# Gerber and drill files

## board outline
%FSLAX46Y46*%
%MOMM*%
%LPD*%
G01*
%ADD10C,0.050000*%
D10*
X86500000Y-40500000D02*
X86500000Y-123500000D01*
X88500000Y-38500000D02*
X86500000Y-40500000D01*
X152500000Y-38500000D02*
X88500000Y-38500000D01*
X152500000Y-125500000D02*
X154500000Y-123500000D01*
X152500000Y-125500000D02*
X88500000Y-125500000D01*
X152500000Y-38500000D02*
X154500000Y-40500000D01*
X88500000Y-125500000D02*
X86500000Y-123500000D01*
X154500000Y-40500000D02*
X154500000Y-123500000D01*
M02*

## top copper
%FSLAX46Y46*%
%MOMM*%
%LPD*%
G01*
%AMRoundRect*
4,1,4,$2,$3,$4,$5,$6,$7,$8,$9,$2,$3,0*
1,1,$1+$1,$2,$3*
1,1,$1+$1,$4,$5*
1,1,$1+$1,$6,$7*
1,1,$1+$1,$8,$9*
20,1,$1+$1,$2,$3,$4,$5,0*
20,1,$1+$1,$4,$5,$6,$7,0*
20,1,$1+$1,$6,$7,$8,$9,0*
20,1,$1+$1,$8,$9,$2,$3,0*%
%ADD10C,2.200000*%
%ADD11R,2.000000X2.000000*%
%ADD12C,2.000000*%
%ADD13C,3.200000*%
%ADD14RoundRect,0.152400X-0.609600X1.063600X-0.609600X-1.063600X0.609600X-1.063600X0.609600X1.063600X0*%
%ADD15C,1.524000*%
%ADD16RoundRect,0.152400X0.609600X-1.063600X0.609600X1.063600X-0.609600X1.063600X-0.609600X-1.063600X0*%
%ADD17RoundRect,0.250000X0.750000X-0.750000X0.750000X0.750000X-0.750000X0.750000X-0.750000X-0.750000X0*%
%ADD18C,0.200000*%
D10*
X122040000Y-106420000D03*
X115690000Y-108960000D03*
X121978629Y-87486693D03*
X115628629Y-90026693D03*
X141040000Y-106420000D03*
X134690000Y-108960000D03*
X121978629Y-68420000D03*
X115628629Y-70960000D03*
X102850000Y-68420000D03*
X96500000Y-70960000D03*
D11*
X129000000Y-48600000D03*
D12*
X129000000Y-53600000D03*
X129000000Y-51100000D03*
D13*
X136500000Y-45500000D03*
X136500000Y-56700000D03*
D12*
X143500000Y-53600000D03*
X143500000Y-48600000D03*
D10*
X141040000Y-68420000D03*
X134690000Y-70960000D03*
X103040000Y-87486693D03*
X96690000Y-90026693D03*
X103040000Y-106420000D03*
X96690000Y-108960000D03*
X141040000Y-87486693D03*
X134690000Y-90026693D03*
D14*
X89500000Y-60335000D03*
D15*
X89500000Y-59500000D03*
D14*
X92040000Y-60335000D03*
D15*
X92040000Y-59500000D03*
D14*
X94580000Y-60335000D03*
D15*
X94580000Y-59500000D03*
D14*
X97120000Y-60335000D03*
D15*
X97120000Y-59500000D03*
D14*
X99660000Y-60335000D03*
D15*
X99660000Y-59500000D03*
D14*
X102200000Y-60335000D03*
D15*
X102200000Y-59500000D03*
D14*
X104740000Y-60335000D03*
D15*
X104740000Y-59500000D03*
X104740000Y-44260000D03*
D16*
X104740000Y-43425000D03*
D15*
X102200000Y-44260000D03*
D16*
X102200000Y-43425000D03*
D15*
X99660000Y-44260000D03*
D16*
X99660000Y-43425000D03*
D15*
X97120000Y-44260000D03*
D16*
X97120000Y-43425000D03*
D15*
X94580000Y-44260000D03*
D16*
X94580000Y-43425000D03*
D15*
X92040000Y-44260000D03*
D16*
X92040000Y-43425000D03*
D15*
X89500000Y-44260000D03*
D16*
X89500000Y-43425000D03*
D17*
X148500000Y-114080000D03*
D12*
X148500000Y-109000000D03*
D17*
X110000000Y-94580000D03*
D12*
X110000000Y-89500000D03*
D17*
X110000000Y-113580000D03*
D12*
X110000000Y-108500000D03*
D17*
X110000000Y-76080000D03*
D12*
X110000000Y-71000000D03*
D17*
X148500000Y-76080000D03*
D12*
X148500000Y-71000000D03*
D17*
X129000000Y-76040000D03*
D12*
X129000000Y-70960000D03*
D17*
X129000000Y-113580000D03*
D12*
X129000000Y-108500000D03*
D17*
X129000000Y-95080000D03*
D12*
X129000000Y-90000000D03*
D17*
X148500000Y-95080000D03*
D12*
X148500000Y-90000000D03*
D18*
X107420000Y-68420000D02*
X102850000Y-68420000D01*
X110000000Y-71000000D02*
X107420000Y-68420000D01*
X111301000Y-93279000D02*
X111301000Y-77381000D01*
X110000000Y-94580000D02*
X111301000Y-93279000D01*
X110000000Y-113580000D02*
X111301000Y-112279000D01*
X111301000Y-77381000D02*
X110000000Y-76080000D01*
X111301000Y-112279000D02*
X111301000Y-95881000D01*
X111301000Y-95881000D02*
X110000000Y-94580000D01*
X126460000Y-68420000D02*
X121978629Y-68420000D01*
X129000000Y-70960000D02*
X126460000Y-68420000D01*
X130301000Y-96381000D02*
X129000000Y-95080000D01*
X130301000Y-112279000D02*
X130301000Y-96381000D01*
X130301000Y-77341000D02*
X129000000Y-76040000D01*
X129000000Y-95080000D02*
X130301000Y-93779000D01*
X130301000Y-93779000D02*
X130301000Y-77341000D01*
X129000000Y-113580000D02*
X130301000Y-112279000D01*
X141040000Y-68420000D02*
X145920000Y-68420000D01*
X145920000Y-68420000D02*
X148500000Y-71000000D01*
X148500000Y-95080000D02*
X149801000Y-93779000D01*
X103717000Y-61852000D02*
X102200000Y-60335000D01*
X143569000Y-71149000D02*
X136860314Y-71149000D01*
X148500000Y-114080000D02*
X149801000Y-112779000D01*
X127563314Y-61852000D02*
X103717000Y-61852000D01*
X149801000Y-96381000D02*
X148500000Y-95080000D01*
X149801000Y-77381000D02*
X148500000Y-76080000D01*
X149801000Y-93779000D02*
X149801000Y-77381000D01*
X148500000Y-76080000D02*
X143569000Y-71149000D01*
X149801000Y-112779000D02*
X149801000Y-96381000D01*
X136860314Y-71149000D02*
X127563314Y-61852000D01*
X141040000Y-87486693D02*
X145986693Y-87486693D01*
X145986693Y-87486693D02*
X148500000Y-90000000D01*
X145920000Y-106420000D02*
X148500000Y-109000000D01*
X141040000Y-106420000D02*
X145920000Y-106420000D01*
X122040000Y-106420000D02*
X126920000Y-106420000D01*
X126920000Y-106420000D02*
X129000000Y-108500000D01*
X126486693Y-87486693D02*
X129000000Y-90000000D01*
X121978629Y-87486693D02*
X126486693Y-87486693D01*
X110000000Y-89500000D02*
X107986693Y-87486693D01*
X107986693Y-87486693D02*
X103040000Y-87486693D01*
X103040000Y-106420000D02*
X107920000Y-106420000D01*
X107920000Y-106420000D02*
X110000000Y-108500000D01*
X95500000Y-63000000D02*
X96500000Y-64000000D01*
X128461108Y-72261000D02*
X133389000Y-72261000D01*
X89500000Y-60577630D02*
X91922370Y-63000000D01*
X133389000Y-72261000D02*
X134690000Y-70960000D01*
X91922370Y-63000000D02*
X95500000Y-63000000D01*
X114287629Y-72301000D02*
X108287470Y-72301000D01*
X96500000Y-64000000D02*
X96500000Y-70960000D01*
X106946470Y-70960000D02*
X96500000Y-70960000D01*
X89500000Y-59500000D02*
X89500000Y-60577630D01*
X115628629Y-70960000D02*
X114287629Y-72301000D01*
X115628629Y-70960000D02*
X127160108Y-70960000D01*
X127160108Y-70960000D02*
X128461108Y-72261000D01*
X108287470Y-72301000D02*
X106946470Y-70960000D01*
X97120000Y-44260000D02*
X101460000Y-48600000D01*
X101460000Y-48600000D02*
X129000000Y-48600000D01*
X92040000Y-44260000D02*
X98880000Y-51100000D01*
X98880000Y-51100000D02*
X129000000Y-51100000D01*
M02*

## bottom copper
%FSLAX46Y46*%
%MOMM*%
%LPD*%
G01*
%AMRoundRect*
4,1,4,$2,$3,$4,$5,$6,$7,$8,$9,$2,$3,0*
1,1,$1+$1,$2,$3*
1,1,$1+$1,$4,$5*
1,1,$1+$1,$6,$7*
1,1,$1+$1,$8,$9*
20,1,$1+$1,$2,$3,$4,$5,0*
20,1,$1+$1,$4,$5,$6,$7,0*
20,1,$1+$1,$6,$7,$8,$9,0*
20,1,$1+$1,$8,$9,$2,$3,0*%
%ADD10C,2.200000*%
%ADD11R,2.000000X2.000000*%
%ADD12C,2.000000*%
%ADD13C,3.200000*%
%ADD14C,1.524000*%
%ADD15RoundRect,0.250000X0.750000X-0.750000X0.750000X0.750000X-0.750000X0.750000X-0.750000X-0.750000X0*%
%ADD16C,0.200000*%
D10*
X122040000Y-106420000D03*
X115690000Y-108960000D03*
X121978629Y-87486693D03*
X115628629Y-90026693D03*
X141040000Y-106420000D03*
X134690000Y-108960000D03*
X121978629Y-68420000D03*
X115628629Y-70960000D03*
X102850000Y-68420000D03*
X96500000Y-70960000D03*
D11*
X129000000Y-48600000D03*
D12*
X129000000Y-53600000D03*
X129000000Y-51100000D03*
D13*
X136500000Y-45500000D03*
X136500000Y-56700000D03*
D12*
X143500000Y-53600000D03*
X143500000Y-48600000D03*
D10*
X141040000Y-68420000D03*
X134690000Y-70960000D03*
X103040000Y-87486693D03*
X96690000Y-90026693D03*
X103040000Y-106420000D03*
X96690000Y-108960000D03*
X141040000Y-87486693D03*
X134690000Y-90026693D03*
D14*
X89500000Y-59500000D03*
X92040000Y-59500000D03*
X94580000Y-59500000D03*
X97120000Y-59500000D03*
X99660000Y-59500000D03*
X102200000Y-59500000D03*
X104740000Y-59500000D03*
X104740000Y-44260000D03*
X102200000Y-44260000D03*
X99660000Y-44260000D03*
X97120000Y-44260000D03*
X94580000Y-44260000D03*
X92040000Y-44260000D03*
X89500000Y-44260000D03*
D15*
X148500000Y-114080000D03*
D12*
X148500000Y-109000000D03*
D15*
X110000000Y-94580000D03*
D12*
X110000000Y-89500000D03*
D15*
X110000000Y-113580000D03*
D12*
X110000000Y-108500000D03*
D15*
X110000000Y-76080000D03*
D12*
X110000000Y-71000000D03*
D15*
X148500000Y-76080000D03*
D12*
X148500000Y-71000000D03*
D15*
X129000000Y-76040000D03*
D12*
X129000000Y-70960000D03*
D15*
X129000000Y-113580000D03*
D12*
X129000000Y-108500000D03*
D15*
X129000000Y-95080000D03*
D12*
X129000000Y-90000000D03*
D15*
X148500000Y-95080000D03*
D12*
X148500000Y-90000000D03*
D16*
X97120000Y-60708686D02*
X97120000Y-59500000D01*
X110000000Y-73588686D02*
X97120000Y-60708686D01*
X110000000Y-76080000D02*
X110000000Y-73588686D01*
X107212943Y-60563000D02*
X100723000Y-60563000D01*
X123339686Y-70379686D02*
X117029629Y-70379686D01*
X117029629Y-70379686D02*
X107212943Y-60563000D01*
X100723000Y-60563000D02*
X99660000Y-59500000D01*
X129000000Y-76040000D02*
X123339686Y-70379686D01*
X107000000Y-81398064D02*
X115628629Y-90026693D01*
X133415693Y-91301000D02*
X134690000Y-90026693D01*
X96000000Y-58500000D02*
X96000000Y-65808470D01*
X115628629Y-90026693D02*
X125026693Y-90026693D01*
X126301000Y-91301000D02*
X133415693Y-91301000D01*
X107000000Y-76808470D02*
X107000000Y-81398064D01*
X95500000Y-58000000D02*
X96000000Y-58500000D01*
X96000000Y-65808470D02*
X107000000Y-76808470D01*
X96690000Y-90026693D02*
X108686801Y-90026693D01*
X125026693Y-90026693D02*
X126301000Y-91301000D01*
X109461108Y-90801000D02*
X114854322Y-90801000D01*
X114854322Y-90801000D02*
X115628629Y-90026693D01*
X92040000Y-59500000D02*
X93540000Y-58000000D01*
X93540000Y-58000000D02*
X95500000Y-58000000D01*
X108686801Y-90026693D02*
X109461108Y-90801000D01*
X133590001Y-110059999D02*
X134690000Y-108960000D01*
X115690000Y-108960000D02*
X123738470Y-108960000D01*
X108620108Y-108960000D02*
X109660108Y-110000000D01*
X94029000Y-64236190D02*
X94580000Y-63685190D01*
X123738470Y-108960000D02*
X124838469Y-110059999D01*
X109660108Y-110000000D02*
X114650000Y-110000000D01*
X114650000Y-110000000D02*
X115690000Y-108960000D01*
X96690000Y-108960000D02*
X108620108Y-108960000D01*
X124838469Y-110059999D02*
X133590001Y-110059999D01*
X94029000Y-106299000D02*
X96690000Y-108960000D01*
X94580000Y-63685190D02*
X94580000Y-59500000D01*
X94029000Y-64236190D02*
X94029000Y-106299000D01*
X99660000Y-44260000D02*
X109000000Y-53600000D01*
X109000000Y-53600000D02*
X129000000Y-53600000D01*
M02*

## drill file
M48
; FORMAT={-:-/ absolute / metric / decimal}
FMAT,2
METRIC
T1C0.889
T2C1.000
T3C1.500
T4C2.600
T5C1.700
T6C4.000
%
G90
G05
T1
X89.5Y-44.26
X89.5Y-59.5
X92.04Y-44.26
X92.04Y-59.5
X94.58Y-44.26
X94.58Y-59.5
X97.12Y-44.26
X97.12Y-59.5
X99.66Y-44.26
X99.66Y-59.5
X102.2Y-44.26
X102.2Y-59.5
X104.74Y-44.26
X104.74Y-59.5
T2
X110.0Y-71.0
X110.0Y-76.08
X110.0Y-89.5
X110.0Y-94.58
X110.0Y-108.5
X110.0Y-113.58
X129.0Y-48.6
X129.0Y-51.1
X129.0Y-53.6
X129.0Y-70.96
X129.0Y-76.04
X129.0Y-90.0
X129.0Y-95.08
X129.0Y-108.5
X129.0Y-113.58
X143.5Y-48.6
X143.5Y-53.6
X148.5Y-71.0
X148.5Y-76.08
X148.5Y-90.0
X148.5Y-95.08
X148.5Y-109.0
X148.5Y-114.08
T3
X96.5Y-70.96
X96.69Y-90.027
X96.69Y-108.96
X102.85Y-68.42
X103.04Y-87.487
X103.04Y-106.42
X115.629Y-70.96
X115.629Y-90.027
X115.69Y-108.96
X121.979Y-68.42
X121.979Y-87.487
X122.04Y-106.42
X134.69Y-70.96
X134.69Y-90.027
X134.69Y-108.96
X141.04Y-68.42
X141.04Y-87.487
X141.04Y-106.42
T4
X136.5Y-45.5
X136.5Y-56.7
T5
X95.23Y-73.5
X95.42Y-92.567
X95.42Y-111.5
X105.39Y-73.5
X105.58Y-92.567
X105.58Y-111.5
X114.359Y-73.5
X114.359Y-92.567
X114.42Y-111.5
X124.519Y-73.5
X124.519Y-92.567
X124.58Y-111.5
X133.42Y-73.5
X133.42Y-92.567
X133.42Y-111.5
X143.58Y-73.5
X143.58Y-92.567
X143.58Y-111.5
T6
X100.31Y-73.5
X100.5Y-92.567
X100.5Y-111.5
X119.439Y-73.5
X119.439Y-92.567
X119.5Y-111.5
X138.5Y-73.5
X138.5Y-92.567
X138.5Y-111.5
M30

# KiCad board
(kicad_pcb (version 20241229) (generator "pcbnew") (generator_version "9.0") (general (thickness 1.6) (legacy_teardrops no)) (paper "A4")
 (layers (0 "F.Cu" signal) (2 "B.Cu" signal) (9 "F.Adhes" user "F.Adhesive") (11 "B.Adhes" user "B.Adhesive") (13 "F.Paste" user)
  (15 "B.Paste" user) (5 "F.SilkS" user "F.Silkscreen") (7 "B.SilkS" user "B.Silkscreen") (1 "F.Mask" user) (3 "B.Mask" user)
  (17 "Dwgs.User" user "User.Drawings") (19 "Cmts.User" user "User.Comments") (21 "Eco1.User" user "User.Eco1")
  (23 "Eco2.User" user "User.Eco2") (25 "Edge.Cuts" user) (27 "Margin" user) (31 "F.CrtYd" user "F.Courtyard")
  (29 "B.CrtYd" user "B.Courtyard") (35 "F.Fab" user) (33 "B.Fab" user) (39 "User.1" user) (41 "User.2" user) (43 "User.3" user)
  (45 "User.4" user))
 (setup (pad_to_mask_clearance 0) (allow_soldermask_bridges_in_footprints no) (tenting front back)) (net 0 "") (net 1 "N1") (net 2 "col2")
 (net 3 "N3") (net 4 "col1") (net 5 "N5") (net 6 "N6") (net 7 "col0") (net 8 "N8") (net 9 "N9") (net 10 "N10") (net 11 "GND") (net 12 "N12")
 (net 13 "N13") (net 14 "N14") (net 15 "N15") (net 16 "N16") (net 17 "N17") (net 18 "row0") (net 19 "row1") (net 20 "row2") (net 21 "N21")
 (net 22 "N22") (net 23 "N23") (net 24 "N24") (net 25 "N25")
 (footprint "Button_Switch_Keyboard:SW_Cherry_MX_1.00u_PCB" (layer "F.Cu") (at 122.04 106.42)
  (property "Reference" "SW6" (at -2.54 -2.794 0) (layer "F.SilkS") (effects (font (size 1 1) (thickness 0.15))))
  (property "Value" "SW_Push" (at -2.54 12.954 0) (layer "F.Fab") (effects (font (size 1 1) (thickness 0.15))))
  (pad "" np_thru_hole circle (at -7.62 5.08) (size 1.7 1.7) (drill 1.7) (layers "*.Cu" "*.Mask"))
  (pad "" np_thru_hole circle (at -2.54 5.08) (size 4 4) (drill 4) (layers "*.Cu" "*.Mask"))
  (pad "" np_thru_hole circle (at 2.54 5.08) (size 1.7 1.7) (drill 1.7) (layers "*.Cu" "*.Mask"))
  (pad "1" thru_hole circle (at 0 0) (size 2.2 2.2) (drill 1.5) (layers "*.Cu" "*.Mask") (remove_unused_layers no) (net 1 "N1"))
  (pad "2" thru_hole circle (at -6.35 2.54) (size 2.2 2.2) (drill 1.5) (layers "*.Cu" "*.Mask") (remove_unused_layers no) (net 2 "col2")))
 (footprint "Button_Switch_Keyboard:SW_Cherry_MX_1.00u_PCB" (layer "F.Cu") (at 121.978629 87.486693)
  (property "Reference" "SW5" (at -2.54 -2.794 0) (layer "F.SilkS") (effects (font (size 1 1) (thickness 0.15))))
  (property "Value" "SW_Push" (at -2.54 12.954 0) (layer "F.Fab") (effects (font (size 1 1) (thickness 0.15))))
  (pad "" np_thru_hole circle (at -7.62 5.08) (size 1.7 1.7) (drill 1.7) (layers "*.Cu" "*.Mask"))
  (pad "" np_thru_hole circle (at -2.54 5.08) (size 4 4) (drill 4) (layers "*.Cu" "*.Mask"))
  (pad "" np_thru_hole circle (at 2.54 5.08) (size 1.7 1.7) (drill 1.7) (layers "*.Cu" "*.Mask"))
  (pad "1" thru_hole circle (at 0 0) (size 2.2 2.2) (drill 1.5) (layers "*.Cu" "*.Mask") (remove_unused_layers no) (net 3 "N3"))
  (pad "2" thru_hole circle (at -6.35 2.54) (size 2.2 2.2) (drill 1.5) (layers "*.Cu" "*.Mask") (remove_unused_layers no) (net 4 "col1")))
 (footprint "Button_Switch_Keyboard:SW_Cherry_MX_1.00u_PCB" (layer "F.Cu") (at 141.04 106.42)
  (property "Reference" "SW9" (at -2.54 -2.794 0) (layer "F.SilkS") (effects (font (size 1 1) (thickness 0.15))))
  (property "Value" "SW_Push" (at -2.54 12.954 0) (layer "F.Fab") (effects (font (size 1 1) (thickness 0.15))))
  (pad "" np_thru_hole circle (at -7.62 5.08) (size 1.7 1.7) (drill 1.7) (layers "*.Cu" "*.Mask"))
  (pad "" np_thru_hole circle (at -2.54 5.08) (size 4 4) (drill 4) (layers "*.Cu" "*.Mask"))
  (pad "" np_thru_hole circle (at 2.54 5.08) (size 1.7 1.7) (drill 1.7) (layers "*.Cu" "*.Mask"))
  (pad "1" thru_hole circle (at 0 0) (size 2.2 2.2) (drill 1.5) (layers "*.Cu" "*.Mask") (remove_unused_layers no) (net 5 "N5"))
  (pad "2" thru_hole circle (at -6.35 2.54) (size 2.2 2.2) (drill 1.5) (layers "*.Cu" "*.Mask") (remove_unused_layers no) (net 2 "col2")))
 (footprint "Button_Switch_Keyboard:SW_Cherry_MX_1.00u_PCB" (layer "F.Cu") (at 121.978629 68.42)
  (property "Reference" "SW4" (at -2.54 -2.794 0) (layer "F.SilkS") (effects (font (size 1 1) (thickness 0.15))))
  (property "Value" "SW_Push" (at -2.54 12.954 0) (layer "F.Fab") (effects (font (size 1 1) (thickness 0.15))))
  (pad "" np_thru_hole circle (at -7.62 5.08) (size 1.7 1.7) (drill 1.7) (layers "*.Cu" "*.Mask"))
  (pad "" np_thru_hole circle (at -2.54 5.08) (size 4 4) (drill 4) (layers "*.Cu" "*.Mask"))
  (pad "" np_thru_hole circle (at 2.54 5.08) (size 1.7 1.7) (drill 1.7) (layers "*.Cu" "*.Mask"))
  (pad "1" thru_hole circle (at 0 0) (size 2.2 2.2) (drill 1.5) (layers "*.Cu" "*.Mask") (remove_unused_layers no) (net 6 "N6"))
  (pad "2" thru_hole circle (at -6.35 2.54) (size 2.2 2.2) (drill 1.5) (layers "*.Cu" "*.Mask") (remove_unused_layers no) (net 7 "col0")))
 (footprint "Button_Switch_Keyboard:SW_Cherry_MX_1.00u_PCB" (layer "F.Cu") (at 102.85 68.42)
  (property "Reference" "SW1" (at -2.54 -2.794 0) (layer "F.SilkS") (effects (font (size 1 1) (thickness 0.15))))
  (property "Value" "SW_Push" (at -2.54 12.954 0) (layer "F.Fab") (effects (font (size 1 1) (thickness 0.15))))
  (pad "" np_thru_hole circle (at -7.62 5.08) (size 1.7 1.7) (drill 1.7) (layers "*.Cu" "*.Mask"))
  (pad "" np_thru_hole circle (at -2.54 5.08) (size 4 4) (drill 4) (layers "*.Cu" "*.Mask"))
  (pad "" np_thru_hole circle (at 2.54 5.08) (size 1.7 1.7) (drill 1.7) (layers "*.Cu" "*.Mask"))
  (pad "1" thru_hole circle (at 0 0) (size 2.2 2.2) (drill 1.5) (layers "*.Cu" "*.Mask") (remove_unused_layers no) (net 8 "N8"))
  (pad "2" thru_hole circle (at -6.35 2.54) (size 2.2 2.2) (drill 1.5) (layers "*.Cu" "*.Mask") (remove_unused_layers no) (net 7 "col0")))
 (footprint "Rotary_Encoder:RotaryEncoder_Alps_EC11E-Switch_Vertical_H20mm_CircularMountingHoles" (layer "F.Cu") (at 129 48.6)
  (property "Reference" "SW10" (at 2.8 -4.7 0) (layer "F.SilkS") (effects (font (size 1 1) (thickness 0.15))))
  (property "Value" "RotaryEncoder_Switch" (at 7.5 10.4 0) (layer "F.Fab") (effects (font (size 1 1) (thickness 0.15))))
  (pad "A" thru_hole rect (at 0 0) (size 2 2) (drill 1) (layers "*.Cu" "*.Mask") (remove_unused_layers no) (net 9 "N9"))
  (pad "B" thru_hole circle (at 0 5) (size 2 2) (drill 1) (layers "*.Cu" "*.Mask") (remove_unused_layers no) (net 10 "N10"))
  (pad "C" thru_hole circle (at 0 2.5) (size 2 2) (drill 1) (layers "*.Cu" "*.Mask") (remove_unused_layers no) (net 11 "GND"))
  (pad "MP" thru_hole circle (at 7.5 -3.1) (size 3.2 3.2) (drill 2.6) (layers "*.Cu" "*.Mask") (remove_unused_layers no))
  (pad "MP" thru_hole circle (at 7.5 8.1) (size 3.2 3.2) (drill 2.6) (layers "*.Cu" "*.Mask") (remove_unused_layers no))
  (pad "S1" thru_hole circle (at 14.5 5) (size 2 2) (drill 1) (layers "*.Cu" "*.Mask") (remove_unused_layers no) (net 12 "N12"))
  (pad "S2" thru_hole circle (at 14.5 0) (size 2 2) (drill 1) (layers "*.Cu" "*.Mask") (remove_unused_layers no) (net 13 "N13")))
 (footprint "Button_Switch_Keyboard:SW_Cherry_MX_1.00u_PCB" (layer "F.Cu") (at 141.04 68.42)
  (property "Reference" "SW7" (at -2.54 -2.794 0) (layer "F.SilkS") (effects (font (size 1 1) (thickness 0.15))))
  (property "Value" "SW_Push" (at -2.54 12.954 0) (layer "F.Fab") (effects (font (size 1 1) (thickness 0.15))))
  (pad "" np_thru_hole circle (at -7.62 5.08) (size 1.7 1.7) (drill 1.7) (layers "*.Cu" "*.Mask"))
  (pad "" np_thru_hole circle (at -2.54 5.08) (size 4 4) (drill 4) (layers "*.Cu" "*.Mask"))
  (pad "" np_thru_hole circle (at 2.54 5.08) (size 1.7 1.7) (drill 1.7) (layers "*.Cu" "*.Mask"))
  (pad "1" thru_hole circle (at 0 0) (size 2.2 2.2) (drill 1.5) (layers "*.Cu" "*.Mask") (remove_unused_layers no) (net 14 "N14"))
  (pad "2" thru_hole circle (at -6.35 2.54) (size 2.2 2.2) (drill 1.5) (layers "*.Cu" "*.Mask") (remove_unused_layers no) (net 7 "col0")))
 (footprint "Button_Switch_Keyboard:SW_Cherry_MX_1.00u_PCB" (layer "F.Cu") (at 103.04 87.486693)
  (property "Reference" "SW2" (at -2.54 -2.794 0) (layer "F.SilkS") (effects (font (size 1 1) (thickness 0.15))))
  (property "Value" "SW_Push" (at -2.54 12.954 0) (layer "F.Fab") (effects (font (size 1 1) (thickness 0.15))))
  (pad "" np_thru_hole circle (at -7.62 5.08) (size 1.7 1.7) (drill 1.7) (layers "*.Cu" "*.Mask"))
  (pad "" np_thru_hole circle (at -2.54 5.08) (size 4 4) (drill 4) (layers "*.Cu" "*.Mask"))
  (pad "" np_thru_hole circle (at 2.54 5.08) (size 1.7 1.7) (drill 1.7) (layers "*.Cu" "*.Mask"))
  (pad "1" thru_hole circle (at 0 0) (size 2.2 2.2) (drill 1.5) (layers "*.Cu" "*.Mask") (remove_unused_layers no) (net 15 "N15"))
  (pad "2" thru_hole circle (at -6.35 2.54) (size 2.2 2.2) (drill 1.5) (layers "*.Cu" "*.Mask") (remove_unused_layers no) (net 4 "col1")))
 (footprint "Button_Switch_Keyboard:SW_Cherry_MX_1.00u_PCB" (layer "F.Cu") (at 103.04 106.42)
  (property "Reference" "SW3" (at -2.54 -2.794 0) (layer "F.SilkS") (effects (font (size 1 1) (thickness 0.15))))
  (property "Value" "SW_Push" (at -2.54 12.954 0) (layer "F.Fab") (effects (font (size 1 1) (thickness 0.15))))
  (pad "" np_thru_hole circle (at -7.62 5.08) (size 1.7 1.7) (drill 1.7) (layers "*.Cu" "*.Mask"))
  (pad "" np_thru_hole circle (at -2.54 5.08) (size 4 4) (drill 4) (layers "*.Cu" "*.Mask"))
  (pad "" np_thru_hole circle (at 2.54 5.08) (size 1.7 1.7) (drill 1.7) (layers "*.Cu" "*.Mask"))
  (pad "1" thru_hole circle (at 0 0) (size 2.2 2.2) (drill 1.5) (layers "*.Cu" "*.Mask") (remove_unused_layers no) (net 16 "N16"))
  (pad "2" thru_hole circle (at -6.35 2.54) (size 2.2 2.2) (drill 1.5) (layers "*.Cu" "*.Mask") (remove_unused_layers no) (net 2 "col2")))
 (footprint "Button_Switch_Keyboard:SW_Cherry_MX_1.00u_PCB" (layer "F.Cu") (at 141.04 87.486693)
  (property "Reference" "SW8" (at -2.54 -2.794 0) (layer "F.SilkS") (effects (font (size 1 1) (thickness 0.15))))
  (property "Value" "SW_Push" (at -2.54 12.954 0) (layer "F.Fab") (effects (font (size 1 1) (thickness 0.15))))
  (pad "" np_thru_hole circle (at -7.62 5.08) (size 1.7 1.7) (drill 1.7) (layers "*.Cu" "*.Mask"))
  (pad "" np_thru_hole circle (at -2.54 5.08) (size 4 4) (drill 4) (layers "*.Cu" "*.Mask"))
  (pad "" np_thru_hole circle (at 2.54 5.08) (size 1.7 1.7) (drill 1.7) (layers "*.Cu" "*.Mask"))
  (pad "1" thru_hole circle (at 0 0) (size 2.2 2.2) (drill 1.5) (layers "*.Cu" "*.Mask") (remove_unused_layers no) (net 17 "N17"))
  (pad "2" thru_hole circle (at -6.35 2.54) (size 2.2 2.2) (drill 1.5) (layers "*.Cu" "*.Mask") (remove_unused_layers no) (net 4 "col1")))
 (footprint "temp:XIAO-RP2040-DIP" (layer "F.Cu") (at 97.12 51.88 90)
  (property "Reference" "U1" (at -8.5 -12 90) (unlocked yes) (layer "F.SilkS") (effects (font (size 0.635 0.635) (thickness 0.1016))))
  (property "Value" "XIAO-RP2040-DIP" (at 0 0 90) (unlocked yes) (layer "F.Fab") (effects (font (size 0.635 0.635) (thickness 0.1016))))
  (pad "1" smd roundrect (at -8.455 -7.62 270) (size 2.432 1.524) (layers "F.Cu" "F.Mask") (roundrect_rratio 0.1) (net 7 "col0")
   (thermal_bridge_angle 45))
  (pad "1" thru_hole circle (at -7.62 -7.62 270) (size 1.524 1.524) (drill 0.889) (layers "*.Cu" "*.Mask") (remove_unused_layers no)
   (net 7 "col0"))
  (pad "2" smd roundrect (at -8.455 -5.08 270) (size 2.432 1.524) (layers "F.Cu" "F.Mask") (roundrect_rratio 0.1) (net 4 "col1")
   (thermal_bridge_angle 45))
  (pad "2" thru_hole circle (at -7.62 -5.08 270) (size 1.524 1.524) (drill 0.889) (layers "*.Cu" "*.Mask") (remove_unused_layers no)
   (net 4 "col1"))
  (pad "3" smd roundrect (at -8.455 -2.54 270) (size 2.432 1.524) (layers "F.Cu" "F.Mask") (roundrect_rratio 0.1) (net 2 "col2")
   (thermal_bridge_angle 45))
  (pad "3" thru_hole circle (at -7.62 -2.54 270) (size 1.524 1.524) (drill 0.889) (layers "*.Cu" "*.Mask") (remove_unused_layers no)
   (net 2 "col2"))
  (pad "4" smd roundrect (at -8.455 0 270) (size 2.432 1.524) (layers "F.Cu" "F.Mask") (roundrect_rratio 0.1) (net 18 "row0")
   (thermal_bridge_angle 45))
  (pad "4" thru_hole circle (at -7.62 0 270) (size 1.524 1.524) (drill 0.889) (layers "*.Cu" "*.Mask") (remove_unused_layers no)
   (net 18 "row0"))
  (pad "5" smd roundrect (at -8.455 2.54 270) (size 2.432 1.524) (layers "F.Cu" "F.Mask") (roundrect_rratio 0.1) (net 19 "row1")
   (thermal_bridge_angle 45))
  (pad "5" thru_hole circle (at -7.62 2.54 270) (size 1.524 1.524) (drill 0.889) (layers "*.Cu" "*.Mask") (remove_unused_layers no)
   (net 19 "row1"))
  (pad "6" smd roundrect (at -8.455 5.08 270) (size 2.432 1.524) (layers "F.Cu" "F.Mask") (roundrect_rratio 0.1) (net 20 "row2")
   (thermal_bridge_angle 45))
  (pad "6" thru_hole circle (at -7.62 5.08 270) (size 1.524 1.524) (drill 0.889) (layers "*.Cu" "*.Mask") (remove_unused_layers no)
   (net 20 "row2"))
  (pad "7" smd roundrect (at -8.455 7.62 270) (size 2.432 1.524) (layers "F.Cu" "F.Mask") (roundrect_rratio 0.1) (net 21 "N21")
   (thermal_bridge_angle 45))
  (pad "7" thru_hole circle (at -7.62 7.62 270) (size 1.524 1.524) (drill 0.889) (layers "*.Cu" "*.Mask") (remove_unused_layers no)
   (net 21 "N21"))
  (pad "8" thru_hole circle (at 7.62 7.62 90) (size 1.524 1.524) (drill 0.889) (layers "*.Cu" "*.Mask") (remove_unused_layers no)
   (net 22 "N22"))
  (pad "8" smd roundrect (at 8.455 7.62 90) (size 2.432 1.524) (layers "F.Cu" "F.Mask") (roundrect_rratio 0.1) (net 22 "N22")
   (thermal_bridge_angle 45))
  (pad "9" thru_hole circle (at 7.62 5.08 90) (size 1.524 1.524) (drill 0.889) (layers "*.Cu" "*.Mask") (remove_unused_layers no)
   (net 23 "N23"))
  (pad "9" smd roundrect (at 8.455 5.08 90) (size 2.432 1.524) (layers "F.Cu" "F.Mask") (roundrect_rratio 0.1) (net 23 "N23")
   (thermal_bridge_angle 45))
  (pad "10" thru_hole circle (at 7.62 2.54 90) (size 1.524 1.524) (drill 0.889) (layers "*.Cu" "*.Mask") (remove_unused_layers no)
   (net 10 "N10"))
  (pad "10" smd roundrect (at 8.455 2.54 90) (size 2.432 1.524) (layers "F.Cu" "F.Mask") (roundrect_rratio 0.1) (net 10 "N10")
   (thermal_bridge_angle 45))
  (pad "11" thru_hole circle (at 7.62 0 90) (size 1.524 1.524) (drill 0.889) (layers "*.Cu" "*.Mask") (remove_unused_layers no) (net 9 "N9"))
  (pad "11" smd roundrect (at 8.455 0 90) (size 2.432 1.524) (layers "F.Cu" "F.Mask") (roundrect_rratio 0.1) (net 9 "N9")
   (thermal_bridge_angle 45))
  (pad "12" thru_hole circle (at 7.62 -2.54 90) (size 1.524 1.524) (drill 0.889) (layers "*.Cu" "*.Mask") (remove_unused_layers no)
   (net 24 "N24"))
  (pad "12" smd roundrect (at 8.455 -2.54 90) (size 2.432 1.524) (layers "F.Cu" "F.Mask") (roundrect_rratio 0.1) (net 24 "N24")
   (thermal_bridge_angle 45))
  (pad "13" thru_hole circle (at 7.62 -5.08 90) (size 1.524 1.524) (drill 0.889) (layers "*.Cu" "*.Mask") (remove_unused_layers no)
   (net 11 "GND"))
  (pad "13" smd roundrect (at 8.455 -5.08 90) (size 2.432 1.524) (layers "F.Cu" "F.Mask") (roundrect_rratio 0.1) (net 11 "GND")
   (thermal_bridge_angle 45))
  (pad "14" thru_hole circle (at 7.62 -7.62 90) (size 1.524 1.524) (drill 0.889) (layers "*.Cu" "*.Mask") (remove_unused_layers no)
   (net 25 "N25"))
  (pad "14" smd roundrect (at 8.455 -7.62 90) (size 2.432 1.524) (layers "F.Cu" "F.Mask") (roundrect_rratio 0.1) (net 25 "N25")
   (thermal_bridge_angle 45)))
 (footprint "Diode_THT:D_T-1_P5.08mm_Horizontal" (layer "B.Cu") (at 148.5 114.08 90)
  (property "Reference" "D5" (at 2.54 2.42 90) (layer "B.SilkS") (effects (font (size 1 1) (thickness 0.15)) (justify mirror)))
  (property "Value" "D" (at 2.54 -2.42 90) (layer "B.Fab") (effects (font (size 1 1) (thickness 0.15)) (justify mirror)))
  (pad "1" thru_hole roundrect (at 0 0 90) (size 2 2) (drill 1) (layers "*.Cu" "*.Mask") (remove_unused_layers no) (roundrect_rratio 0.125)
   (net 20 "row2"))
  (pad "2" thru_hole circle (at 5.08 0 90) (size 2 2) (drill 1) (layers "*.Cu" "*.Mask") (remove_unused_layers no) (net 5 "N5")))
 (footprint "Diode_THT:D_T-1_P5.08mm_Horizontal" (layer "B.Cu") (at 110 94.58 90)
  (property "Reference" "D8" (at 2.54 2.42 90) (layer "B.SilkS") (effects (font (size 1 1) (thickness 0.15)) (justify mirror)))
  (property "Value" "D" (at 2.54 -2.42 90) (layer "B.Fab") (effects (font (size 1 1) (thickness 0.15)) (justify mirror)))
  (pad "1" thru_hole roundrect (at 0 0 90) (size 2 2) (drill 1) (layers "*.Cu" "*.Mask") (remove_unused_layers no) (roundrect_rratio 0.125)
   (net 18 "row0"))
  (pad "2" thru_hole circle (at 5.08 0 90) (size 2 2) (drill 1) (layers "*.Cu" "*.Mask") (remove_unused_layers no) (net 15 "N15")))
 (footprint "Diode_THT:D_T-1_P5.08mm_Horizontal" (layer "B.Cu") (at 110 113.58 90)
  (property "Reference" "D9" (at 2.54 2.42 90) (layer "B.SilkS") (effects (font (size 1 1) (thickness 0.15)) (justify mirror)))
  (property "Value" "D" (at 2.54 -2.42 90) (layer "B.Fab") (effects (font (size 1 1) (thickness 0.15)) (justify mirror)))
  (pad "1" thru_hole roundrect (at 0 0 90) (size 2 2) (drill 1) (layers "*.Cu" "*.Mask") (remove_unused_layers no) (roundrect_rratio 0.125)
   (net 18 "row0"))
  (pad "2" thru_hole circle (at 5.08 0 90) (size 2 2) (drill 1) (layers "*.Cu" "*.Mask") (remove_unused_layers no) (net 16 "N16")))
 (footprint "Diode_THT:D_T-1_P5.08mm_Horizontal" (layer "B.Cu") (at 110 76.08 90)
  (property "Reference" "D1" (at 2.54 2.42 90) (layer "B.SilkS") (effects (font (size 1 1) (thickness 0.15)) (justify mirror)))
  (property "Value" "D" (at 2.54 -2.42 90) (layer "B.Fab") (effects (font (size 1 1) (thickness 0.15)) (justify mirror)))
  (pad "1" thru_hole roundrect (at 0 0 90) (size 2 2) (drill 1) (layers "*.Cu" "*.Mask") (remove_unused_layers no) (roundrect_rratio 0.125)
   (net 18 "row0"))
  (pad "2" thru_hole circle (at 5.08 0 90) (size 2 2) (drill 1) (layers "*.Cu" "*.Mask") (remove_unused_layers no) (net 8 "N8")))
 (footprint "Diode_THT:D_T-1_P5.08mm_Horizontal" (layer "B.Cu") (at 148.5 76.08 90)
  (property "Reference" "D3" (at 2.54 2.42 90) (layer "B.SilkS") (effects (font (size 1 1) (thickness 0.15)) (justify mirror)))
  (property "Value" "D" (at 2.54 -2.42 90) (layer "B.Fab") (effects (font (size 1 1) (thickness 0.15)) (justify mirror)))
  (pad "1" thru_hole roundrect (at 0 0 90) (size 2 2) (drill 1) (layers "*.Cu" "*.Mask") (remove_unused_layers no) (roundrect_rratio 0.125)
   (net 20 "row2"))
  (pad "2" thru_hole circle (at 5.08 0 90) (size 2 2) (drill 1) (layers "*.Cu" "*.Mask") (remove_unused_layers no) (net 14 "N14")))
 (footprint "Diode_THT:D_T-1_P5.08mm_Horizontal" (layer "B.Cu") (at 129 76.04 90)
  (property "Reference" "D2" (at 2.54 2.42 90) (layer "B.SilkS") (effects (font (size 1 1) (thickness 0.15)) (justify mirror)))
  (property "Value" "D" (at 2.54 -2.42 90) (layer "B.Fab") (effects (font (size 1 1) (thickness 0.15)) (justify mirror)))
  (pad "1" thru_hole roundrect (at 0 0 90) (size 2 2) (drill 1) (layers "*.Cu" "*.Mask") (remove_unused_layers no) (roundrect_rratio 0.125)
   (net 19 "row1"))
  (pad "2" thru_hole circle (at 5.08 0 90) (size 2 2) (drill 1) (layers "*.Cu" "*.Mask") (remove_unused_layers no) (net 6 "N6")))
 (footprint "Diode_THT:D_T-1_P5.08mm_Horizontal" (layer "B.Cu") (at 129 113.58 90)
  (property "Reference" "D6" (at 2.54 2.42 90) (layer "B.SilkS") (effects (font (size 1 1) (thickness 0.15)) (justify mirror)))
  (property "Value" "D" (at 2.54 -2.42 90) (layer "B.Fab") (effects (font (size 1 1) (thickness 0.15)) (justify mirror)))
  (pad "1" thru_hole roundrect (at 0 0 90) (size 2 2) (drill 1) (layers "*.Cu" "*.Mask") (remove_unused_layers no) (roundrect_rratio 0.125)
   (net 19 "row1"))
  (pad "2" thru_hole circle (at 5.08 0 90) (size 2 2) (drill 1) (layers "*.Cu" "*.Mask") (remove_unused_layers no) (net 1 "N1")))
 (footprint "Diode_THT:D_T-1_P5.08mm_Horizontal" (layer "B.Cu") (at 129 95.08 90)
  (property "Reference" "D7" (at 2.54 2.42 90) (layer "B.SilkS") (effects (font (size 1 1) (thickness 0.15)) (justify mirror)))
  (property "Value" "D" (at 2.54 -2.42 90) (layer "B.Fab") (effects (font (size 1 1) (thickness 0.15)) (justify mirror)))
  (pad "1" thru_hole roundrect (at 0 0 90) (size 2 2) (drill 1) (layers "*.Cu" "*.Mask") (remove_unused_layers no) (roundrect_rratio 0.125)
   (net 19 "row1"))
  (pad "2" thru_hole circle (at 5.08 0 90) (size 2 2) (drill 1) (layers "*.Cu" "*.Mask") (remove_unused_layers no) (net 3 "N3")))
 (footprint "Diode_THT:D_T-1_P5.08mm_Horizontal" (layer "B.Cu") (at 148.5 95.08 90)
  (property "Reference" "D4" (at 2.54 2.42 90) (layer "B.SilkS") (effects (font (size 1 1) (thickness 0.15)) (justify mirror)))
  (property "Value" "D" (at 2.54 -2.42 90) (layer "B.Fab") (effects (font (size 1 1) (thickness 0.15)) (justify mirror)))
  (pad "1" thru_hole roundrect (at 0 0 90) (size 2 2) (drill 1) (layers "*.Cu" "*.Mask") (remove_unused_layers no) (roundrect_rratio 0.125)
   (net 20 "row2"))
  (pad "2" thru_hole circle (at 5.08 0 90) (size 2 2) (drill 1) (layers "*.Cu" "*.Mask") (remove_unused_layers no) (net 17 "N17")))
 (gr_line (start 86.5 40.5) (end 86.5 123.5) (stroke (width 0.05) (type default)) (layer "Edge.Cuts"))
 (gr_line (start 88.5 38.5) (end 86.5 40.5) (stroke (width 0.05) (type default)) (layer "Edge.Cuts"))
 (gr_line (start 152.5 38.5) (end 88.5 38.5) (stroke (width 0.05) (type default)) (layer "Edge.Cuts"))
 (gr_line (start 152.5 125.5) (end 154.5 123.5) (stroke (width 0.05) (type default)) (layer "Edge.Cuts"))
 (gr_line (start 152.5 125.5) (end 88.5 125.5) (stroke (width 0.05) (type default)) (layer "Edge.Cuts"))
 (gr_line (start 152.5 38.5) (end 154.5 40.5) (stroke (width 0.05) (type default)) (layer "Edge.Cuts"))
 (gr_line (start 88.5 125.5) (end 86.5 123.5) (stroke (width 0.05) (type default)) (layer "Edge.Cuts"))
 (gr_line (start 154.5 40.5) (end 154.5 123.5) (stroke (width 0.05) (type default)) (layer "Edge.Cuts"))
 (segment (start 107.42 68.42) (end 102.85 68.42) (width 0.2) (layer "F.Cu") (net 8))
 (segment (start 110 71) (end 107.42 68.42) (width 0.2) (layer "F.Cu") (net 8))
 (segment (start 111.301 93.279) (end 111.301 77.381) (width 0.2) (layer "F.Cu") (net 18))
 (segment (start 110 94.58) (end 111.301 93.279) (width 0.2) (layer "F.Cu") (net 18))
 (segment (start 110 113.58) (end 111.301 112.279) (width 0.2) (layer "F.Cu") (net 18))
 (segment (start 111.301 77.381) (end 110 76.08) (width 0.2) (layer "F.Cu") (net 18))
 (segment (start 111.301 112.279) (end 111.301 95.881) (width 0.2) (layer "F.Cu") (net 18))
 (segment (start 111.301 95.881) (end 110 94.58) (width 0.2) (layer "F.Cu") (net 18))
 (segment (start 97.12 60.708686) (end 97.12 59.5) (width 0.2) (layer "B.Cu") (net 18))
 (segment (start 110 73.588686) (end 97.12 60.708686) (width 0.2) (layer "B.Cu") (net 18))
 (segment (start 110 76.08) (end 110 73.588686) (width 0.2) (layer "B.Cu") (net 18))
 (segment (start 126.46 68.42) (end 121.978629 68.42) (width 0.2) (layer "F.Cu") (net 6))
 (segment (start 129 70.96) (end 126.46 68.42) (width 0.2) (layer "F.Cu") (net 6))
 (segment (start 130.301 96.381) (end 129 95.08) (width 0.2) (layer "F.Cu") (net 19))
 (segment (start 130.301 112.279) (end 130.301 96.381) (width 0.2) (layer "F.Cu") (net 19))
 (segment (start 130.301 77.341) (end 129 76.04) (width 0.2) (layer "F.Cu") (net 19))
 (segment (start 129 95.08) (end 130.301 93.779) (width 0.2) (layer "F.Cu") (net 19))
 (segment (start 130.301 93.779) (end 130.301 77.341) (width 0.2) (layer "F.Cu") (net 19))
 (segment (start 129 113.58) (end 130.301 112.279) (width 0.2) (layer "F.Cu") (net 19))
 (segment (start 107.212943 60.563) (end 100.723 60.563) (width 0.2) (layer "B.Cu") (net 19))
 (segment (start 123.339686 70.379686) (end 117.029629 70.379686) (width 0.2) (layer "B.Cu") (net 19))
 (segment (start 117.029629 70.379686) (end 107.212943 60.563) (width 0.2) (layer "B.Cu") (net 19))
 (segment (start 100.723 60.563) (end 99.66 59.5) (width 0.2) (layer "B.Cu") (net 19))
 (segment (start 129 76.04) (end 123.339686 70.379686) (width 0.2) (layer "B.Cu") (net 19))
 (segment (start 141.04 68.42) (end 145.92 68.42) (width 0.2) (layer "F.Cu") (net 14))
 (segment (start 145.92 68.42) (end 148.5 71) (width 0.2) (layer "F.Cu") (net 14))
 (segment (start 148.5 95.08) (end 149.801 93.779) (width 0.2) (layer "F.Cu") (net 20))
 (segment (start 103.717 61.852) (end 102.2 60.335) (width 0.2) (layer "F.Cu") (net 20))
 (segment (start 143.569 71.149) (end 136.860314 71.149) (width 0.2) (layer "F.Cu") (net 20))
 (segment (start 148.5 114.08) (end 149.801 112.779) (width 0.2) (layer "F.Cu") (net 20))
 (segment (start 127.563314 61.852) (end 103.717 61.852) (width 0.2) (layer "F.Cu") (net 20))
 (segment (start 149.801 96.381) (end 148.5 95.08) (width 0.2) (layer "F.Cu") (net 20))
 (segment (start 149.801 77.381) (end 148.5 76.08) (width 0.2) (layer "F.Cu") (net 20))
 (segment (start 149.801 93.779) (end 149.801 77.381) (width 0.2) (layer "F.Cu") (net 20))
 (segment (start 148.5 76.08) (end 143.569 71.149) (width 0.2) (layer "F.Cu") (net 20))
 (segment (start 149.801 112.779) (end 149.801 96.381) (width 0.2) (layer "F.Cu") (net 20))
 (segment (start 136.860314 71.149) (end 127.563314 61.852) (width 0.2) (layer "F.Cu") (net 20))
 (segment (start 141.04 87.486693) (end 145.986693 87.486693) (width 0.2) (layer "F.Cu") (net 17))
 (segment (start 145.986693 87.486693) (end 148.5 90) (width 0.2) (layer "F.Cu") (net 17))
 (segment (start 145.92 106.42) (end 148.5 109) (width 0.2) (layer "F.Cu") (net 5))
 (segment (start 141.04 106.42) (end 145.92 106.42) (width 0.2) (layer "F.Cu") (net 5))
 (segment (start 122.04 106.42) (end 126.92 106.42) (width 0.2) (layer "F.Cu") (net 1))
 (segment (start 126.92 106.42) (end 129 108.5) (width 0.2) (layer "F.Cu") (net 1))
 (segment (start 126.486693 87.486693) (end 129 90) (width 0.2) (layer "F.Cu") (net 3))
 (segment (start 121.978629 87.486693) (end 126.486693 87.486693) (width 0.2) (layer "F.Cu") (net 3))
 (segment (start 110 89.5) (end 107.986693 87.486693) (width 0.2) (layer "F.Cu") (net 15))
 (segment (start 107.986693 87.486693) (end 103.04 87.486693) (width 0.2) (layer "F.Cu") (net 15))
 (segment (start 103.04 106.42) (end 107.92 106.42) (width 0.2) (layer "F.Cu") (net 16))
 (segment (start 107.92 106.42) (end 110 108.5) (width 0.2) (layer "F.Cu") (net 16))
 (segment (start 95.5 63) (end 96.5 64) (width 0.2) (layer "F.Cu") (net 7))
 (segment (start 128.461108 72.261) (end 133.389 72.261) (width 0.2) (layer "F.Cu") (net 7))
 (segment (start 89.5 60.57763) (end 91.92237 63) (width 0.2) (layer "F.Cu") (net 7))
 (segment (start 133.389 72.261) (end 134.69 70.96) (width 0.2) (layer "F.Cu") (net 7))
 (segment (start 91.92237 63) (end 95.5 63) (width 0.2) (layer "F.Cu") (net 7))
 (segment (start 114.287629 72.301) (end 108.28747 72.301) (width 0.2) (layer "F.Cu") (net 7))
 (segment (start 96.5 64) (end 96.5 70.96) (width 0.2) (layer "F.Cu") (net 7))
 (segment (start 106.94647 70.96) (end 96.5 70.96) (width 0.2) (layer "F.Cu") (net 7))
 (segment (start 89.5 59.5) (end 89.5 60.57763) (width 0.2) (layer "F.Cu") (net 7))
 (segment (start 115.628629 70.96) (end 114.287629 72.301) (width 0.2) (layer "F.Cu") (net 7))
 (segment (start 115.628629 70.96) (end 127.160108 70.96) (width 0.2) (layer "F.Cu") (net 7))
 (segment (start 127.160108 70.96) (end 128.461108 72.261) (width 0.2) (layer "F.Cu") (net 7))
 (segment (start 108.28747 72.301) (end 106.94647 70.96) (width 0.2) (layer "F.Cu") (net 7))
 (segment (start 107 81.398064) (end 115.628629 90.026693) (width 0.2) (layer "B.Cu") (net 4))
 (segment (start 133.415693 91.301) (end 134.69 90.026693) (width 0.2) (layer "B.Cu") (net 4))
 (segment (start 96 58.5) (end 96 65.80847) (width 0.2) (layer "B.Cu") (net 4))
 (segment (start 115.628629 90.026693) (end 125.026693 90.026693) (width 0.2) (layer "B.Cu") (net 4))
 (segment (start 126.301 91.301) (end 133.415693 91.301) (width 0.2) (layer "B.Cu") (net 4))
 (segment (start 107 76.80847) (end 107 81.398064) (width 0.2) (layer "B.Cu") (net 4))
 (segment (start 95.5 58) (end 96 58.5) (width 0.2) (layer "B.Cu") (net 4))
 (segment (start 96 65.80847) (end 107 76.80847) (width 0.2) (layer "B.Cu") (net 4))
 (segment (start 96.69 90.026693) (end 108.686801 90.026693) (width 0.2) (layer "B.Cu") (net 4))
 (segment (start 125.026693 90.026693) (end 126.301 91.301) (width 0.2) (layer "B.Cu") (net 4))
 (segment (start 109.461108 90.801) (end 114.854322 90.801) (width 0.2) (layer "B.Cu") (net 4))
 (segment (start 114.854322 90.801) (end 115.628629 90.026693) (width 0.2) (layer "B.Cu") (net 4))
 (segment (start 92.04 59.5) (end 93.54 58) (width 0.2) (layer "B.Cu") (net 4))
 (segment (start 93.54 58) (end 95.5 58) (width 0.2) (layer "B.Cu") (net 4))
 (segment (start 108.686801 90.026693) (end 109.461108 90.801) (width 0.2) (layer "B.Cu") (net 4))
 (segment (start 133.590001 110.059999) (end 134.69 108.96) (width 0.2) (layer "B.Cu") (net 2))
 (segment (start 115.69 108.96) (end 123.73847 108.96) (width 0.2) (layer "B.Cu") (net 2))
 (segment (start 108.620108 108.96) (end 109.660108 110) (width 0.2) (layer "B.Cu") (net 2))
 (segment (start 94.029 64.23619) (end 94.58 63.68519) (width 0.2) (layer "B.Cu") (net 2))
 (segment (start 123.73847 108.96) (end 124.838469 110.059999) (width 0.2) (layer "B.Cu") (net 2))
 (segment (start 109.660108 110) (end 114.65 110) (width 0.2) (layer "B.Cu") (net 2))
 (segment (start 114.65 110) (end 115.69 108.96) (width 0.2) (layer "B.Cu") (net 2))
 (segment (start 96.69 108.96) (end 108.620108 108.96) (width 0.2) (layer "B.Cu") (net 2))
 (segment (start 124.838469 110.059999) (end 133.590001 110.059999) (width 0.2) (layer "B.Cu") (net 2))
 (segment (start 94.029 106.299) (end 96.69 108.96) (width 0.2) (layer "B.Cu") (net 2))
 (segment (start 94.58 63.68519) (end 94.58 59.5) (width 0.2) (layer "B.Cu") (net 2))
 (segment (start 94.029 64.23619) (end 94.029 106.299) (width 0.2) (layer "B.Cu") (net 2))
 (segment (start 97.12 44.26) (end 101.46 48.6) (width 0.2) (layer "F.Cu") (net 9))
 (segment (start 101.46 48.6) (end 129 48.6) (width 0.2) (layer "F.Cu") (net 9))
 (segment (start 99.66 44.26) (end 109 53.6) (width 0.2) (layer "B.Cu") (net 10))
 (segment (start 109 53.6) (end 129 53.6) (width 0.2) (layer "B.Cu") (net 10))
 (segment (start 92.04 44.26) (end 98.88 51.1) (width 0.2) (layer "F.Cu") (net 11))
 (segment (start 98.88 51.1) (end 129 51.1) (width 0.2) (layer "F.Cu") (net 11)))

